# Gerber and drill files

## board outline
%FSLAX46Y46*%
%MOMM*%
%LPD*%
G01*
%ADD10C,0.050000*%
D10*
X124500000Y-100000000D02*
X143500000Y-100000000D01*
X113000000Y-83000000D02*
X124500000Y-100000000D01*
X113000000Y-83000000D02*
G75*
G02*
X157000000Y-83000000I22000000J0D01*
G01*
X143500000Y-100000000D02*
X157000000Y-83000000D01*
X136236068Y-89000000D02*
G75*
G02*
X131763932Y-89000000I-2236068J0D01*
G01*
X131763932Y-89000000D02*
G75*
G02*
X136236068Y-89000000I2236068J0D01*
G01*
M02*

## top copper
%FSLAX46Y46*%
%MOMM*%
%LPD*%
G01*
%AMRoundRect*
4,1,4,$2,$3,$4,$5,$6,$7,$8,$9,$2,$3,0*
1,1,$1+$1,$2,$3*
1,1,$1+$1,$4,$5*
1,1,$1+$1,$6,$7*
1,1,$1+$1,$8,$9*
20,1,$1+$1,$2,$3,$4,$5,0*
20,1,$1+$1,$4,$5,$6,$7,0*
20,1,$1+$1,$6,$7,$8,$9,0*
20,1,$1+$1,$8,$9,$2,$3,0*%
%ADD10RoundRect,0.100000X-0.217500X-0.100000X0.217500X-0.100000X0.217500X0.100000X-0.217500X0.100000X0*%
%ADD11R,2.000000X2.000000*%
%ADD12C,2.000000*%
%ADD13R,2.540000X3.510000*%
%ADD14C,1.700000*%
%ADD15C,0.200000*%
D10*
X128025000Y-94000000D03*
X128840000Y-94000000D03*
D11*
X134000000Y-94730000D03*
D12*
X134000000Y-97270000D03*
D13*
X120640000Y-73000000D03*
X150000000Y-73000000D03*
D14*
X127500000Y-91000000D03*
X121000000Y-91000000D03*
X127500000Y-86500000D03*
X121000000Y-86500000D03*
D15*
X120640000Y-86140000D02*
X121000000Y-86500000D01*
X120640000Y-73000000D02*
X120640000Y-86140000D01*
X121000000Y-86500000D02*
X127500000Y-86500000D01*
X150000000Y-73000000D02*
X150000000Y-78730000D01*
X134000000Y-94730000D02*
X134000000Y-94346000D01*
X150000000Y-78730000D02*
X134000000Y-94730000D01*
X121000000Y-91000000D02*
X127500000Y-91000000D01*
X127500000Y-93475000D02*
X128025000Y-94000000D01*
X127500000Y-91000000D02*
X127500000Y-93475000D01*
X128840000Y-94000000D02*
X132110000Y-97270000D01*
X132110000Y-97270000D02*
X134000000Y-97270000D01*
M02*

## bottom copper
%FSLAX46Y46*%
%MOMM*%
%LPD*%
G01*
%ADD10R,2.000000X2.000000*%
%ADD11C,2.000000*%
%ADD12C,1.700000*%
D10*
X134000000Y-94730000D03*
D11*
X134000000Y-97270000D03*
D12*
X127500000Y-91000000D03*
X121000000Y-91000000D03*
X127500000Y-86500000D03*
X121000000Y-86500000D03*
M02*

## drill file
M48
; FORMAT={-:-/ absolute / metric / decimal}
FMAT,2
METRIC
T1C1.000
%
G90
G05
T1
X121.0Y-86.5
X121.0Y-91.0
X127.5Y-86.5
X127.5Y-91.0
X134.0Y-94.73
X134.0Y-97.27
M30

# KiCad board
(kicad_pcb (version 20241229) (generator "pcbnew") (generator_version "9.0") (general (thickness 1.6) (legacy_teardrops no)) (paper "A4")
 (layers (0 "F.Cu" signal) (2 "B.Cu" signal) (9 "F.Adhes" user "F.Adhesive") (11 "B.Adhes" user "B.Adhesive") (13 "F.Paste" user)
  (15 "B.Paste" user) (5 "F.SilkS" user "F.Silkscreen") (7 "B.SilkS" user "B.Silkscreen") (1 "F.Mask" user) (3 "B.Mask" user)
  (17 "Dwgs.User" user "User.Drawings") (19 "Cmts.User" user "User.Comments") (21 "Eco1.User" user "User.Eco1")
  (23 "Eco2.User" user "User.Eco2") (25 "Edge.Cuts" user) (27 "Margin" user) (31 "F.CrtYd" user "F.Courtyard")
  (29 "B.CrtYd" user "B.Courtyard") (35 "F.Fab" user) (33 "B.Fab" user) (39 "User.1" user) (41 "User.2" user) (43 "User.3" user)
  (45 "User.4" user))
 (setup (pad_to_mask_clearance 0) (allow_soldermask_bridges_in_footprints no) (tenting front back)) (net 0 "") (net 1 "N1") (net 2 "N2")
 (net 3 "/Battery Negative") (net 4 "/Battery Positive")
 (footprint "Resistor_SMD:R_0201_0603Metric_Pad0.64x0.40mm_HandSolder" (layer "F.Cu") (at 128.4325 94)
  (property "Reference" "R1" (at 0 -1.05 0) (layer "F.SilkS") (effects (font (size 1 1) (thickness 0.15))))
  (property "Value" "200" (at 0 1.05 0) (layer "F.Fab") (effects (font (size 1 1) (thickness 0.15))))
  (pad "" smd roundrect (at -0.4325 0) (size 0.458 0.36) (layers "F.Paste") (roundrect_rratio 0.25))
  (pad "" smd roundrect (at 0.4325 0) (size 0.458 0.36) (layers "F.Paste") (roundrect_rratio 0.25))
  (pad "1" smd roundrect (at -0.4075 0) (size 0.635 0.4) (layers "F.Cu" "F.Mask") (roundrect_rratio 0.25) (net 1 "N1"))
  (pad "2" smd roundrect (at 0.4075 0) (size 0.635 0.4) (layers "F.Cu" "F.Mask") (roundrect_rratio 0.25) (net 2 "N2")))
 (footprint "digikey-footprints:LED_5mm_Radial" (layer "F.Cu") (at 134 97.27 -90)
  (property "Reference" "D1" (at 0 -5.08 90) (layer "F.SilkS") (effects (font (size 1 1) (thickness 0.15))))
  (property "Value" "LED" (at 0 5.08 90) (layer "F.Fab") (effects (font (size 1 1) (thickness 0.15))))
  (pad "1" thru_hole rect (at -2.54 0 270) (size 2 2) (drill 1) (layers "*.Cu" "*.Mask") (remove_unused_layers no)
   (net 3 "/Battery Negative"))
  (pad "2" thru_hole circle (at 0 0 270) (size 2 2) (drill 1) (layers "*.Cu" "*.Mask") (remove_unused_layers no) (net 2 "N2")))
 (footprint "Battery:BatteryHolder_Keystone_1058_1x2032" (layer "F.Cu") (at 135.32 73)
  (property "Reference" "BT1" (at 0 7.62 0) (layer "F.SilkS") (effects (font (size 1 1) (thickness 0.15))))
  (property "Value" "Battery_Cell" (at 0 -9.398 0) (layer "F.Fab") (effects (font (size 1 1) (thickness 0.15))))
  (pad "1" smd rect (at -14.68 0) (size 2.54 3.51) (layers "F.Cu" "F.Mask" "F.Paste") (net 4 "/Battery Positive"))
  (pad "2" smd rect (at 14.68 0) (size 2.54 3.51) (layers "F.Cu" "F.Mask" "F.Paste") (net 3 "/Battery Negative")))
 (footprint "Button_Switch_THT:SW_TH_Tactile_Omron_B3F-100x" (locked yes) (layer "F.Cu") (at 127.5 91 180)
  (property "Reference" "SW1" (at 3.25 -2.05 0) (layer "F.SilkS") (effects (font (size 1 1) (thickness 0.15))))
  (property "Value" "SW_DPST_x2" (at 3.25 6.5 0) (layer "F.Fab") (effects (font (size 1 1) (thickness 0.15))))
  (pad "1" thru_hole circle (at 0 0 180) (size 1.7 1.7) (drill 1) (layers "*.Cu" "*.Mask") (remove_unused_layers no) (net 1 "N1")
   (thermal_bridge_angle 90))
  (pad "1" thru_hole circle (at 6.5 0 180) (size 1.7 1.7) (drill 1) (layers "*.Cu" "*.Mask") (remove_unused_layers no) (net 1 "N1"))
  (pad "2" thru_hole circle (at 0 4.5 180) (size 1.7 1.7) (drill 1) (layers "*.Cu" "*.Mask") (remove_unused_layers no)
   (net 4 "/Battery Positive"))
  (pad "2" thru_hole circle (at 6.5 4.5 180) (size 1.7 1.7) (drill 1) (layers "*.Cu" "*.Mask") (remove_unused_layers no)
   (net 4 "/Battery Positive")))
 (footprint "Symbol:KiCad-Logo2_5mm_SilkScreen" (layer "B.Cu") (at 134.005617 79.375 180)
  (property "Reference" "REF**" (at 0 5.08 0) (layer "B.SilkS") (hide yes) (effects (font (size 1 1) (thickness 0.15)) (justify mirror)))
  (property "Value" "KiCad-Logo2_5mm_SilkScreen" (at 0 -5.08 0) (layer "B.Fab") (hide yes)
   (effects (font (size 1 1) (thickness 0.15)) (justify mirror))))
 (gr_line (start 124.5 100) (end 143.5 100) (stroke (width 0.05) (type default)) (layer "Edge.Cuts"))
 (gr_line (start 113 83) (end 124.5 100) (stroke (width 0.05) (type default)) (layer "Edge.Cuts"))
 (gr_arc (start 113 83) (mid 135 61) (end 157 83) (stroke (width 0.05) (type default)) (layer "Edge.Cuts"))
 (gr_line (start 143.5 100) (end 157 83) (stroke (width 0.05) (type default)) (layer "Edge.Cuts"))
 (gr_circle (center 134 89) (end 135 87) (stroke (width 0.05) (type default)) (fill no) (layer "Edge.Cuts"))
 (segment (start 120.64 86.14) (end 121 86.5) (width 0.2) (layer "F.Cu") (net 4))
 (segment (start 120.64 73) (end 120.64 86.14) (width 0.2) (layer "F.Cu") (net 4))
 (segment (start 121 86.5) (end 127.5 86.5) (width 0.2) (layer "F.Cu") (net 4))
 (segment (start 150 73) (end 150 78.73) (width 0.2) (layer "F.Cu") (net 3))
 (segment (start 134 94.73) (end 134 94.346) (width 0.2) (layer "F.Cu") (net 3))
 (segment (start 150 78.73) (end 134 94.73) (width 0.2) (layer "F.Cu") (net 3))
 (segment (start 121 91) (end 127.5 91) (width 0.2) (layer "F.Cu") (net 1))
 (segment (start 127.5 93.475) (end 128.025 94) (width 0.2) (layer "F.Cu") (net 1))
 (segment (start 127.5 91) (end 127.5 93.475) (width 0.2) (layer "F.Cu") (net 1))
 (segment (start 128.84 94) (end 132.11 97.27) (width 0.2) (layer "F.Cu") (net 2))
 (segment (start 132.11 97.27) (end 134 97.27) (width 0.2) (layer "F.Cu") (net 2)))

